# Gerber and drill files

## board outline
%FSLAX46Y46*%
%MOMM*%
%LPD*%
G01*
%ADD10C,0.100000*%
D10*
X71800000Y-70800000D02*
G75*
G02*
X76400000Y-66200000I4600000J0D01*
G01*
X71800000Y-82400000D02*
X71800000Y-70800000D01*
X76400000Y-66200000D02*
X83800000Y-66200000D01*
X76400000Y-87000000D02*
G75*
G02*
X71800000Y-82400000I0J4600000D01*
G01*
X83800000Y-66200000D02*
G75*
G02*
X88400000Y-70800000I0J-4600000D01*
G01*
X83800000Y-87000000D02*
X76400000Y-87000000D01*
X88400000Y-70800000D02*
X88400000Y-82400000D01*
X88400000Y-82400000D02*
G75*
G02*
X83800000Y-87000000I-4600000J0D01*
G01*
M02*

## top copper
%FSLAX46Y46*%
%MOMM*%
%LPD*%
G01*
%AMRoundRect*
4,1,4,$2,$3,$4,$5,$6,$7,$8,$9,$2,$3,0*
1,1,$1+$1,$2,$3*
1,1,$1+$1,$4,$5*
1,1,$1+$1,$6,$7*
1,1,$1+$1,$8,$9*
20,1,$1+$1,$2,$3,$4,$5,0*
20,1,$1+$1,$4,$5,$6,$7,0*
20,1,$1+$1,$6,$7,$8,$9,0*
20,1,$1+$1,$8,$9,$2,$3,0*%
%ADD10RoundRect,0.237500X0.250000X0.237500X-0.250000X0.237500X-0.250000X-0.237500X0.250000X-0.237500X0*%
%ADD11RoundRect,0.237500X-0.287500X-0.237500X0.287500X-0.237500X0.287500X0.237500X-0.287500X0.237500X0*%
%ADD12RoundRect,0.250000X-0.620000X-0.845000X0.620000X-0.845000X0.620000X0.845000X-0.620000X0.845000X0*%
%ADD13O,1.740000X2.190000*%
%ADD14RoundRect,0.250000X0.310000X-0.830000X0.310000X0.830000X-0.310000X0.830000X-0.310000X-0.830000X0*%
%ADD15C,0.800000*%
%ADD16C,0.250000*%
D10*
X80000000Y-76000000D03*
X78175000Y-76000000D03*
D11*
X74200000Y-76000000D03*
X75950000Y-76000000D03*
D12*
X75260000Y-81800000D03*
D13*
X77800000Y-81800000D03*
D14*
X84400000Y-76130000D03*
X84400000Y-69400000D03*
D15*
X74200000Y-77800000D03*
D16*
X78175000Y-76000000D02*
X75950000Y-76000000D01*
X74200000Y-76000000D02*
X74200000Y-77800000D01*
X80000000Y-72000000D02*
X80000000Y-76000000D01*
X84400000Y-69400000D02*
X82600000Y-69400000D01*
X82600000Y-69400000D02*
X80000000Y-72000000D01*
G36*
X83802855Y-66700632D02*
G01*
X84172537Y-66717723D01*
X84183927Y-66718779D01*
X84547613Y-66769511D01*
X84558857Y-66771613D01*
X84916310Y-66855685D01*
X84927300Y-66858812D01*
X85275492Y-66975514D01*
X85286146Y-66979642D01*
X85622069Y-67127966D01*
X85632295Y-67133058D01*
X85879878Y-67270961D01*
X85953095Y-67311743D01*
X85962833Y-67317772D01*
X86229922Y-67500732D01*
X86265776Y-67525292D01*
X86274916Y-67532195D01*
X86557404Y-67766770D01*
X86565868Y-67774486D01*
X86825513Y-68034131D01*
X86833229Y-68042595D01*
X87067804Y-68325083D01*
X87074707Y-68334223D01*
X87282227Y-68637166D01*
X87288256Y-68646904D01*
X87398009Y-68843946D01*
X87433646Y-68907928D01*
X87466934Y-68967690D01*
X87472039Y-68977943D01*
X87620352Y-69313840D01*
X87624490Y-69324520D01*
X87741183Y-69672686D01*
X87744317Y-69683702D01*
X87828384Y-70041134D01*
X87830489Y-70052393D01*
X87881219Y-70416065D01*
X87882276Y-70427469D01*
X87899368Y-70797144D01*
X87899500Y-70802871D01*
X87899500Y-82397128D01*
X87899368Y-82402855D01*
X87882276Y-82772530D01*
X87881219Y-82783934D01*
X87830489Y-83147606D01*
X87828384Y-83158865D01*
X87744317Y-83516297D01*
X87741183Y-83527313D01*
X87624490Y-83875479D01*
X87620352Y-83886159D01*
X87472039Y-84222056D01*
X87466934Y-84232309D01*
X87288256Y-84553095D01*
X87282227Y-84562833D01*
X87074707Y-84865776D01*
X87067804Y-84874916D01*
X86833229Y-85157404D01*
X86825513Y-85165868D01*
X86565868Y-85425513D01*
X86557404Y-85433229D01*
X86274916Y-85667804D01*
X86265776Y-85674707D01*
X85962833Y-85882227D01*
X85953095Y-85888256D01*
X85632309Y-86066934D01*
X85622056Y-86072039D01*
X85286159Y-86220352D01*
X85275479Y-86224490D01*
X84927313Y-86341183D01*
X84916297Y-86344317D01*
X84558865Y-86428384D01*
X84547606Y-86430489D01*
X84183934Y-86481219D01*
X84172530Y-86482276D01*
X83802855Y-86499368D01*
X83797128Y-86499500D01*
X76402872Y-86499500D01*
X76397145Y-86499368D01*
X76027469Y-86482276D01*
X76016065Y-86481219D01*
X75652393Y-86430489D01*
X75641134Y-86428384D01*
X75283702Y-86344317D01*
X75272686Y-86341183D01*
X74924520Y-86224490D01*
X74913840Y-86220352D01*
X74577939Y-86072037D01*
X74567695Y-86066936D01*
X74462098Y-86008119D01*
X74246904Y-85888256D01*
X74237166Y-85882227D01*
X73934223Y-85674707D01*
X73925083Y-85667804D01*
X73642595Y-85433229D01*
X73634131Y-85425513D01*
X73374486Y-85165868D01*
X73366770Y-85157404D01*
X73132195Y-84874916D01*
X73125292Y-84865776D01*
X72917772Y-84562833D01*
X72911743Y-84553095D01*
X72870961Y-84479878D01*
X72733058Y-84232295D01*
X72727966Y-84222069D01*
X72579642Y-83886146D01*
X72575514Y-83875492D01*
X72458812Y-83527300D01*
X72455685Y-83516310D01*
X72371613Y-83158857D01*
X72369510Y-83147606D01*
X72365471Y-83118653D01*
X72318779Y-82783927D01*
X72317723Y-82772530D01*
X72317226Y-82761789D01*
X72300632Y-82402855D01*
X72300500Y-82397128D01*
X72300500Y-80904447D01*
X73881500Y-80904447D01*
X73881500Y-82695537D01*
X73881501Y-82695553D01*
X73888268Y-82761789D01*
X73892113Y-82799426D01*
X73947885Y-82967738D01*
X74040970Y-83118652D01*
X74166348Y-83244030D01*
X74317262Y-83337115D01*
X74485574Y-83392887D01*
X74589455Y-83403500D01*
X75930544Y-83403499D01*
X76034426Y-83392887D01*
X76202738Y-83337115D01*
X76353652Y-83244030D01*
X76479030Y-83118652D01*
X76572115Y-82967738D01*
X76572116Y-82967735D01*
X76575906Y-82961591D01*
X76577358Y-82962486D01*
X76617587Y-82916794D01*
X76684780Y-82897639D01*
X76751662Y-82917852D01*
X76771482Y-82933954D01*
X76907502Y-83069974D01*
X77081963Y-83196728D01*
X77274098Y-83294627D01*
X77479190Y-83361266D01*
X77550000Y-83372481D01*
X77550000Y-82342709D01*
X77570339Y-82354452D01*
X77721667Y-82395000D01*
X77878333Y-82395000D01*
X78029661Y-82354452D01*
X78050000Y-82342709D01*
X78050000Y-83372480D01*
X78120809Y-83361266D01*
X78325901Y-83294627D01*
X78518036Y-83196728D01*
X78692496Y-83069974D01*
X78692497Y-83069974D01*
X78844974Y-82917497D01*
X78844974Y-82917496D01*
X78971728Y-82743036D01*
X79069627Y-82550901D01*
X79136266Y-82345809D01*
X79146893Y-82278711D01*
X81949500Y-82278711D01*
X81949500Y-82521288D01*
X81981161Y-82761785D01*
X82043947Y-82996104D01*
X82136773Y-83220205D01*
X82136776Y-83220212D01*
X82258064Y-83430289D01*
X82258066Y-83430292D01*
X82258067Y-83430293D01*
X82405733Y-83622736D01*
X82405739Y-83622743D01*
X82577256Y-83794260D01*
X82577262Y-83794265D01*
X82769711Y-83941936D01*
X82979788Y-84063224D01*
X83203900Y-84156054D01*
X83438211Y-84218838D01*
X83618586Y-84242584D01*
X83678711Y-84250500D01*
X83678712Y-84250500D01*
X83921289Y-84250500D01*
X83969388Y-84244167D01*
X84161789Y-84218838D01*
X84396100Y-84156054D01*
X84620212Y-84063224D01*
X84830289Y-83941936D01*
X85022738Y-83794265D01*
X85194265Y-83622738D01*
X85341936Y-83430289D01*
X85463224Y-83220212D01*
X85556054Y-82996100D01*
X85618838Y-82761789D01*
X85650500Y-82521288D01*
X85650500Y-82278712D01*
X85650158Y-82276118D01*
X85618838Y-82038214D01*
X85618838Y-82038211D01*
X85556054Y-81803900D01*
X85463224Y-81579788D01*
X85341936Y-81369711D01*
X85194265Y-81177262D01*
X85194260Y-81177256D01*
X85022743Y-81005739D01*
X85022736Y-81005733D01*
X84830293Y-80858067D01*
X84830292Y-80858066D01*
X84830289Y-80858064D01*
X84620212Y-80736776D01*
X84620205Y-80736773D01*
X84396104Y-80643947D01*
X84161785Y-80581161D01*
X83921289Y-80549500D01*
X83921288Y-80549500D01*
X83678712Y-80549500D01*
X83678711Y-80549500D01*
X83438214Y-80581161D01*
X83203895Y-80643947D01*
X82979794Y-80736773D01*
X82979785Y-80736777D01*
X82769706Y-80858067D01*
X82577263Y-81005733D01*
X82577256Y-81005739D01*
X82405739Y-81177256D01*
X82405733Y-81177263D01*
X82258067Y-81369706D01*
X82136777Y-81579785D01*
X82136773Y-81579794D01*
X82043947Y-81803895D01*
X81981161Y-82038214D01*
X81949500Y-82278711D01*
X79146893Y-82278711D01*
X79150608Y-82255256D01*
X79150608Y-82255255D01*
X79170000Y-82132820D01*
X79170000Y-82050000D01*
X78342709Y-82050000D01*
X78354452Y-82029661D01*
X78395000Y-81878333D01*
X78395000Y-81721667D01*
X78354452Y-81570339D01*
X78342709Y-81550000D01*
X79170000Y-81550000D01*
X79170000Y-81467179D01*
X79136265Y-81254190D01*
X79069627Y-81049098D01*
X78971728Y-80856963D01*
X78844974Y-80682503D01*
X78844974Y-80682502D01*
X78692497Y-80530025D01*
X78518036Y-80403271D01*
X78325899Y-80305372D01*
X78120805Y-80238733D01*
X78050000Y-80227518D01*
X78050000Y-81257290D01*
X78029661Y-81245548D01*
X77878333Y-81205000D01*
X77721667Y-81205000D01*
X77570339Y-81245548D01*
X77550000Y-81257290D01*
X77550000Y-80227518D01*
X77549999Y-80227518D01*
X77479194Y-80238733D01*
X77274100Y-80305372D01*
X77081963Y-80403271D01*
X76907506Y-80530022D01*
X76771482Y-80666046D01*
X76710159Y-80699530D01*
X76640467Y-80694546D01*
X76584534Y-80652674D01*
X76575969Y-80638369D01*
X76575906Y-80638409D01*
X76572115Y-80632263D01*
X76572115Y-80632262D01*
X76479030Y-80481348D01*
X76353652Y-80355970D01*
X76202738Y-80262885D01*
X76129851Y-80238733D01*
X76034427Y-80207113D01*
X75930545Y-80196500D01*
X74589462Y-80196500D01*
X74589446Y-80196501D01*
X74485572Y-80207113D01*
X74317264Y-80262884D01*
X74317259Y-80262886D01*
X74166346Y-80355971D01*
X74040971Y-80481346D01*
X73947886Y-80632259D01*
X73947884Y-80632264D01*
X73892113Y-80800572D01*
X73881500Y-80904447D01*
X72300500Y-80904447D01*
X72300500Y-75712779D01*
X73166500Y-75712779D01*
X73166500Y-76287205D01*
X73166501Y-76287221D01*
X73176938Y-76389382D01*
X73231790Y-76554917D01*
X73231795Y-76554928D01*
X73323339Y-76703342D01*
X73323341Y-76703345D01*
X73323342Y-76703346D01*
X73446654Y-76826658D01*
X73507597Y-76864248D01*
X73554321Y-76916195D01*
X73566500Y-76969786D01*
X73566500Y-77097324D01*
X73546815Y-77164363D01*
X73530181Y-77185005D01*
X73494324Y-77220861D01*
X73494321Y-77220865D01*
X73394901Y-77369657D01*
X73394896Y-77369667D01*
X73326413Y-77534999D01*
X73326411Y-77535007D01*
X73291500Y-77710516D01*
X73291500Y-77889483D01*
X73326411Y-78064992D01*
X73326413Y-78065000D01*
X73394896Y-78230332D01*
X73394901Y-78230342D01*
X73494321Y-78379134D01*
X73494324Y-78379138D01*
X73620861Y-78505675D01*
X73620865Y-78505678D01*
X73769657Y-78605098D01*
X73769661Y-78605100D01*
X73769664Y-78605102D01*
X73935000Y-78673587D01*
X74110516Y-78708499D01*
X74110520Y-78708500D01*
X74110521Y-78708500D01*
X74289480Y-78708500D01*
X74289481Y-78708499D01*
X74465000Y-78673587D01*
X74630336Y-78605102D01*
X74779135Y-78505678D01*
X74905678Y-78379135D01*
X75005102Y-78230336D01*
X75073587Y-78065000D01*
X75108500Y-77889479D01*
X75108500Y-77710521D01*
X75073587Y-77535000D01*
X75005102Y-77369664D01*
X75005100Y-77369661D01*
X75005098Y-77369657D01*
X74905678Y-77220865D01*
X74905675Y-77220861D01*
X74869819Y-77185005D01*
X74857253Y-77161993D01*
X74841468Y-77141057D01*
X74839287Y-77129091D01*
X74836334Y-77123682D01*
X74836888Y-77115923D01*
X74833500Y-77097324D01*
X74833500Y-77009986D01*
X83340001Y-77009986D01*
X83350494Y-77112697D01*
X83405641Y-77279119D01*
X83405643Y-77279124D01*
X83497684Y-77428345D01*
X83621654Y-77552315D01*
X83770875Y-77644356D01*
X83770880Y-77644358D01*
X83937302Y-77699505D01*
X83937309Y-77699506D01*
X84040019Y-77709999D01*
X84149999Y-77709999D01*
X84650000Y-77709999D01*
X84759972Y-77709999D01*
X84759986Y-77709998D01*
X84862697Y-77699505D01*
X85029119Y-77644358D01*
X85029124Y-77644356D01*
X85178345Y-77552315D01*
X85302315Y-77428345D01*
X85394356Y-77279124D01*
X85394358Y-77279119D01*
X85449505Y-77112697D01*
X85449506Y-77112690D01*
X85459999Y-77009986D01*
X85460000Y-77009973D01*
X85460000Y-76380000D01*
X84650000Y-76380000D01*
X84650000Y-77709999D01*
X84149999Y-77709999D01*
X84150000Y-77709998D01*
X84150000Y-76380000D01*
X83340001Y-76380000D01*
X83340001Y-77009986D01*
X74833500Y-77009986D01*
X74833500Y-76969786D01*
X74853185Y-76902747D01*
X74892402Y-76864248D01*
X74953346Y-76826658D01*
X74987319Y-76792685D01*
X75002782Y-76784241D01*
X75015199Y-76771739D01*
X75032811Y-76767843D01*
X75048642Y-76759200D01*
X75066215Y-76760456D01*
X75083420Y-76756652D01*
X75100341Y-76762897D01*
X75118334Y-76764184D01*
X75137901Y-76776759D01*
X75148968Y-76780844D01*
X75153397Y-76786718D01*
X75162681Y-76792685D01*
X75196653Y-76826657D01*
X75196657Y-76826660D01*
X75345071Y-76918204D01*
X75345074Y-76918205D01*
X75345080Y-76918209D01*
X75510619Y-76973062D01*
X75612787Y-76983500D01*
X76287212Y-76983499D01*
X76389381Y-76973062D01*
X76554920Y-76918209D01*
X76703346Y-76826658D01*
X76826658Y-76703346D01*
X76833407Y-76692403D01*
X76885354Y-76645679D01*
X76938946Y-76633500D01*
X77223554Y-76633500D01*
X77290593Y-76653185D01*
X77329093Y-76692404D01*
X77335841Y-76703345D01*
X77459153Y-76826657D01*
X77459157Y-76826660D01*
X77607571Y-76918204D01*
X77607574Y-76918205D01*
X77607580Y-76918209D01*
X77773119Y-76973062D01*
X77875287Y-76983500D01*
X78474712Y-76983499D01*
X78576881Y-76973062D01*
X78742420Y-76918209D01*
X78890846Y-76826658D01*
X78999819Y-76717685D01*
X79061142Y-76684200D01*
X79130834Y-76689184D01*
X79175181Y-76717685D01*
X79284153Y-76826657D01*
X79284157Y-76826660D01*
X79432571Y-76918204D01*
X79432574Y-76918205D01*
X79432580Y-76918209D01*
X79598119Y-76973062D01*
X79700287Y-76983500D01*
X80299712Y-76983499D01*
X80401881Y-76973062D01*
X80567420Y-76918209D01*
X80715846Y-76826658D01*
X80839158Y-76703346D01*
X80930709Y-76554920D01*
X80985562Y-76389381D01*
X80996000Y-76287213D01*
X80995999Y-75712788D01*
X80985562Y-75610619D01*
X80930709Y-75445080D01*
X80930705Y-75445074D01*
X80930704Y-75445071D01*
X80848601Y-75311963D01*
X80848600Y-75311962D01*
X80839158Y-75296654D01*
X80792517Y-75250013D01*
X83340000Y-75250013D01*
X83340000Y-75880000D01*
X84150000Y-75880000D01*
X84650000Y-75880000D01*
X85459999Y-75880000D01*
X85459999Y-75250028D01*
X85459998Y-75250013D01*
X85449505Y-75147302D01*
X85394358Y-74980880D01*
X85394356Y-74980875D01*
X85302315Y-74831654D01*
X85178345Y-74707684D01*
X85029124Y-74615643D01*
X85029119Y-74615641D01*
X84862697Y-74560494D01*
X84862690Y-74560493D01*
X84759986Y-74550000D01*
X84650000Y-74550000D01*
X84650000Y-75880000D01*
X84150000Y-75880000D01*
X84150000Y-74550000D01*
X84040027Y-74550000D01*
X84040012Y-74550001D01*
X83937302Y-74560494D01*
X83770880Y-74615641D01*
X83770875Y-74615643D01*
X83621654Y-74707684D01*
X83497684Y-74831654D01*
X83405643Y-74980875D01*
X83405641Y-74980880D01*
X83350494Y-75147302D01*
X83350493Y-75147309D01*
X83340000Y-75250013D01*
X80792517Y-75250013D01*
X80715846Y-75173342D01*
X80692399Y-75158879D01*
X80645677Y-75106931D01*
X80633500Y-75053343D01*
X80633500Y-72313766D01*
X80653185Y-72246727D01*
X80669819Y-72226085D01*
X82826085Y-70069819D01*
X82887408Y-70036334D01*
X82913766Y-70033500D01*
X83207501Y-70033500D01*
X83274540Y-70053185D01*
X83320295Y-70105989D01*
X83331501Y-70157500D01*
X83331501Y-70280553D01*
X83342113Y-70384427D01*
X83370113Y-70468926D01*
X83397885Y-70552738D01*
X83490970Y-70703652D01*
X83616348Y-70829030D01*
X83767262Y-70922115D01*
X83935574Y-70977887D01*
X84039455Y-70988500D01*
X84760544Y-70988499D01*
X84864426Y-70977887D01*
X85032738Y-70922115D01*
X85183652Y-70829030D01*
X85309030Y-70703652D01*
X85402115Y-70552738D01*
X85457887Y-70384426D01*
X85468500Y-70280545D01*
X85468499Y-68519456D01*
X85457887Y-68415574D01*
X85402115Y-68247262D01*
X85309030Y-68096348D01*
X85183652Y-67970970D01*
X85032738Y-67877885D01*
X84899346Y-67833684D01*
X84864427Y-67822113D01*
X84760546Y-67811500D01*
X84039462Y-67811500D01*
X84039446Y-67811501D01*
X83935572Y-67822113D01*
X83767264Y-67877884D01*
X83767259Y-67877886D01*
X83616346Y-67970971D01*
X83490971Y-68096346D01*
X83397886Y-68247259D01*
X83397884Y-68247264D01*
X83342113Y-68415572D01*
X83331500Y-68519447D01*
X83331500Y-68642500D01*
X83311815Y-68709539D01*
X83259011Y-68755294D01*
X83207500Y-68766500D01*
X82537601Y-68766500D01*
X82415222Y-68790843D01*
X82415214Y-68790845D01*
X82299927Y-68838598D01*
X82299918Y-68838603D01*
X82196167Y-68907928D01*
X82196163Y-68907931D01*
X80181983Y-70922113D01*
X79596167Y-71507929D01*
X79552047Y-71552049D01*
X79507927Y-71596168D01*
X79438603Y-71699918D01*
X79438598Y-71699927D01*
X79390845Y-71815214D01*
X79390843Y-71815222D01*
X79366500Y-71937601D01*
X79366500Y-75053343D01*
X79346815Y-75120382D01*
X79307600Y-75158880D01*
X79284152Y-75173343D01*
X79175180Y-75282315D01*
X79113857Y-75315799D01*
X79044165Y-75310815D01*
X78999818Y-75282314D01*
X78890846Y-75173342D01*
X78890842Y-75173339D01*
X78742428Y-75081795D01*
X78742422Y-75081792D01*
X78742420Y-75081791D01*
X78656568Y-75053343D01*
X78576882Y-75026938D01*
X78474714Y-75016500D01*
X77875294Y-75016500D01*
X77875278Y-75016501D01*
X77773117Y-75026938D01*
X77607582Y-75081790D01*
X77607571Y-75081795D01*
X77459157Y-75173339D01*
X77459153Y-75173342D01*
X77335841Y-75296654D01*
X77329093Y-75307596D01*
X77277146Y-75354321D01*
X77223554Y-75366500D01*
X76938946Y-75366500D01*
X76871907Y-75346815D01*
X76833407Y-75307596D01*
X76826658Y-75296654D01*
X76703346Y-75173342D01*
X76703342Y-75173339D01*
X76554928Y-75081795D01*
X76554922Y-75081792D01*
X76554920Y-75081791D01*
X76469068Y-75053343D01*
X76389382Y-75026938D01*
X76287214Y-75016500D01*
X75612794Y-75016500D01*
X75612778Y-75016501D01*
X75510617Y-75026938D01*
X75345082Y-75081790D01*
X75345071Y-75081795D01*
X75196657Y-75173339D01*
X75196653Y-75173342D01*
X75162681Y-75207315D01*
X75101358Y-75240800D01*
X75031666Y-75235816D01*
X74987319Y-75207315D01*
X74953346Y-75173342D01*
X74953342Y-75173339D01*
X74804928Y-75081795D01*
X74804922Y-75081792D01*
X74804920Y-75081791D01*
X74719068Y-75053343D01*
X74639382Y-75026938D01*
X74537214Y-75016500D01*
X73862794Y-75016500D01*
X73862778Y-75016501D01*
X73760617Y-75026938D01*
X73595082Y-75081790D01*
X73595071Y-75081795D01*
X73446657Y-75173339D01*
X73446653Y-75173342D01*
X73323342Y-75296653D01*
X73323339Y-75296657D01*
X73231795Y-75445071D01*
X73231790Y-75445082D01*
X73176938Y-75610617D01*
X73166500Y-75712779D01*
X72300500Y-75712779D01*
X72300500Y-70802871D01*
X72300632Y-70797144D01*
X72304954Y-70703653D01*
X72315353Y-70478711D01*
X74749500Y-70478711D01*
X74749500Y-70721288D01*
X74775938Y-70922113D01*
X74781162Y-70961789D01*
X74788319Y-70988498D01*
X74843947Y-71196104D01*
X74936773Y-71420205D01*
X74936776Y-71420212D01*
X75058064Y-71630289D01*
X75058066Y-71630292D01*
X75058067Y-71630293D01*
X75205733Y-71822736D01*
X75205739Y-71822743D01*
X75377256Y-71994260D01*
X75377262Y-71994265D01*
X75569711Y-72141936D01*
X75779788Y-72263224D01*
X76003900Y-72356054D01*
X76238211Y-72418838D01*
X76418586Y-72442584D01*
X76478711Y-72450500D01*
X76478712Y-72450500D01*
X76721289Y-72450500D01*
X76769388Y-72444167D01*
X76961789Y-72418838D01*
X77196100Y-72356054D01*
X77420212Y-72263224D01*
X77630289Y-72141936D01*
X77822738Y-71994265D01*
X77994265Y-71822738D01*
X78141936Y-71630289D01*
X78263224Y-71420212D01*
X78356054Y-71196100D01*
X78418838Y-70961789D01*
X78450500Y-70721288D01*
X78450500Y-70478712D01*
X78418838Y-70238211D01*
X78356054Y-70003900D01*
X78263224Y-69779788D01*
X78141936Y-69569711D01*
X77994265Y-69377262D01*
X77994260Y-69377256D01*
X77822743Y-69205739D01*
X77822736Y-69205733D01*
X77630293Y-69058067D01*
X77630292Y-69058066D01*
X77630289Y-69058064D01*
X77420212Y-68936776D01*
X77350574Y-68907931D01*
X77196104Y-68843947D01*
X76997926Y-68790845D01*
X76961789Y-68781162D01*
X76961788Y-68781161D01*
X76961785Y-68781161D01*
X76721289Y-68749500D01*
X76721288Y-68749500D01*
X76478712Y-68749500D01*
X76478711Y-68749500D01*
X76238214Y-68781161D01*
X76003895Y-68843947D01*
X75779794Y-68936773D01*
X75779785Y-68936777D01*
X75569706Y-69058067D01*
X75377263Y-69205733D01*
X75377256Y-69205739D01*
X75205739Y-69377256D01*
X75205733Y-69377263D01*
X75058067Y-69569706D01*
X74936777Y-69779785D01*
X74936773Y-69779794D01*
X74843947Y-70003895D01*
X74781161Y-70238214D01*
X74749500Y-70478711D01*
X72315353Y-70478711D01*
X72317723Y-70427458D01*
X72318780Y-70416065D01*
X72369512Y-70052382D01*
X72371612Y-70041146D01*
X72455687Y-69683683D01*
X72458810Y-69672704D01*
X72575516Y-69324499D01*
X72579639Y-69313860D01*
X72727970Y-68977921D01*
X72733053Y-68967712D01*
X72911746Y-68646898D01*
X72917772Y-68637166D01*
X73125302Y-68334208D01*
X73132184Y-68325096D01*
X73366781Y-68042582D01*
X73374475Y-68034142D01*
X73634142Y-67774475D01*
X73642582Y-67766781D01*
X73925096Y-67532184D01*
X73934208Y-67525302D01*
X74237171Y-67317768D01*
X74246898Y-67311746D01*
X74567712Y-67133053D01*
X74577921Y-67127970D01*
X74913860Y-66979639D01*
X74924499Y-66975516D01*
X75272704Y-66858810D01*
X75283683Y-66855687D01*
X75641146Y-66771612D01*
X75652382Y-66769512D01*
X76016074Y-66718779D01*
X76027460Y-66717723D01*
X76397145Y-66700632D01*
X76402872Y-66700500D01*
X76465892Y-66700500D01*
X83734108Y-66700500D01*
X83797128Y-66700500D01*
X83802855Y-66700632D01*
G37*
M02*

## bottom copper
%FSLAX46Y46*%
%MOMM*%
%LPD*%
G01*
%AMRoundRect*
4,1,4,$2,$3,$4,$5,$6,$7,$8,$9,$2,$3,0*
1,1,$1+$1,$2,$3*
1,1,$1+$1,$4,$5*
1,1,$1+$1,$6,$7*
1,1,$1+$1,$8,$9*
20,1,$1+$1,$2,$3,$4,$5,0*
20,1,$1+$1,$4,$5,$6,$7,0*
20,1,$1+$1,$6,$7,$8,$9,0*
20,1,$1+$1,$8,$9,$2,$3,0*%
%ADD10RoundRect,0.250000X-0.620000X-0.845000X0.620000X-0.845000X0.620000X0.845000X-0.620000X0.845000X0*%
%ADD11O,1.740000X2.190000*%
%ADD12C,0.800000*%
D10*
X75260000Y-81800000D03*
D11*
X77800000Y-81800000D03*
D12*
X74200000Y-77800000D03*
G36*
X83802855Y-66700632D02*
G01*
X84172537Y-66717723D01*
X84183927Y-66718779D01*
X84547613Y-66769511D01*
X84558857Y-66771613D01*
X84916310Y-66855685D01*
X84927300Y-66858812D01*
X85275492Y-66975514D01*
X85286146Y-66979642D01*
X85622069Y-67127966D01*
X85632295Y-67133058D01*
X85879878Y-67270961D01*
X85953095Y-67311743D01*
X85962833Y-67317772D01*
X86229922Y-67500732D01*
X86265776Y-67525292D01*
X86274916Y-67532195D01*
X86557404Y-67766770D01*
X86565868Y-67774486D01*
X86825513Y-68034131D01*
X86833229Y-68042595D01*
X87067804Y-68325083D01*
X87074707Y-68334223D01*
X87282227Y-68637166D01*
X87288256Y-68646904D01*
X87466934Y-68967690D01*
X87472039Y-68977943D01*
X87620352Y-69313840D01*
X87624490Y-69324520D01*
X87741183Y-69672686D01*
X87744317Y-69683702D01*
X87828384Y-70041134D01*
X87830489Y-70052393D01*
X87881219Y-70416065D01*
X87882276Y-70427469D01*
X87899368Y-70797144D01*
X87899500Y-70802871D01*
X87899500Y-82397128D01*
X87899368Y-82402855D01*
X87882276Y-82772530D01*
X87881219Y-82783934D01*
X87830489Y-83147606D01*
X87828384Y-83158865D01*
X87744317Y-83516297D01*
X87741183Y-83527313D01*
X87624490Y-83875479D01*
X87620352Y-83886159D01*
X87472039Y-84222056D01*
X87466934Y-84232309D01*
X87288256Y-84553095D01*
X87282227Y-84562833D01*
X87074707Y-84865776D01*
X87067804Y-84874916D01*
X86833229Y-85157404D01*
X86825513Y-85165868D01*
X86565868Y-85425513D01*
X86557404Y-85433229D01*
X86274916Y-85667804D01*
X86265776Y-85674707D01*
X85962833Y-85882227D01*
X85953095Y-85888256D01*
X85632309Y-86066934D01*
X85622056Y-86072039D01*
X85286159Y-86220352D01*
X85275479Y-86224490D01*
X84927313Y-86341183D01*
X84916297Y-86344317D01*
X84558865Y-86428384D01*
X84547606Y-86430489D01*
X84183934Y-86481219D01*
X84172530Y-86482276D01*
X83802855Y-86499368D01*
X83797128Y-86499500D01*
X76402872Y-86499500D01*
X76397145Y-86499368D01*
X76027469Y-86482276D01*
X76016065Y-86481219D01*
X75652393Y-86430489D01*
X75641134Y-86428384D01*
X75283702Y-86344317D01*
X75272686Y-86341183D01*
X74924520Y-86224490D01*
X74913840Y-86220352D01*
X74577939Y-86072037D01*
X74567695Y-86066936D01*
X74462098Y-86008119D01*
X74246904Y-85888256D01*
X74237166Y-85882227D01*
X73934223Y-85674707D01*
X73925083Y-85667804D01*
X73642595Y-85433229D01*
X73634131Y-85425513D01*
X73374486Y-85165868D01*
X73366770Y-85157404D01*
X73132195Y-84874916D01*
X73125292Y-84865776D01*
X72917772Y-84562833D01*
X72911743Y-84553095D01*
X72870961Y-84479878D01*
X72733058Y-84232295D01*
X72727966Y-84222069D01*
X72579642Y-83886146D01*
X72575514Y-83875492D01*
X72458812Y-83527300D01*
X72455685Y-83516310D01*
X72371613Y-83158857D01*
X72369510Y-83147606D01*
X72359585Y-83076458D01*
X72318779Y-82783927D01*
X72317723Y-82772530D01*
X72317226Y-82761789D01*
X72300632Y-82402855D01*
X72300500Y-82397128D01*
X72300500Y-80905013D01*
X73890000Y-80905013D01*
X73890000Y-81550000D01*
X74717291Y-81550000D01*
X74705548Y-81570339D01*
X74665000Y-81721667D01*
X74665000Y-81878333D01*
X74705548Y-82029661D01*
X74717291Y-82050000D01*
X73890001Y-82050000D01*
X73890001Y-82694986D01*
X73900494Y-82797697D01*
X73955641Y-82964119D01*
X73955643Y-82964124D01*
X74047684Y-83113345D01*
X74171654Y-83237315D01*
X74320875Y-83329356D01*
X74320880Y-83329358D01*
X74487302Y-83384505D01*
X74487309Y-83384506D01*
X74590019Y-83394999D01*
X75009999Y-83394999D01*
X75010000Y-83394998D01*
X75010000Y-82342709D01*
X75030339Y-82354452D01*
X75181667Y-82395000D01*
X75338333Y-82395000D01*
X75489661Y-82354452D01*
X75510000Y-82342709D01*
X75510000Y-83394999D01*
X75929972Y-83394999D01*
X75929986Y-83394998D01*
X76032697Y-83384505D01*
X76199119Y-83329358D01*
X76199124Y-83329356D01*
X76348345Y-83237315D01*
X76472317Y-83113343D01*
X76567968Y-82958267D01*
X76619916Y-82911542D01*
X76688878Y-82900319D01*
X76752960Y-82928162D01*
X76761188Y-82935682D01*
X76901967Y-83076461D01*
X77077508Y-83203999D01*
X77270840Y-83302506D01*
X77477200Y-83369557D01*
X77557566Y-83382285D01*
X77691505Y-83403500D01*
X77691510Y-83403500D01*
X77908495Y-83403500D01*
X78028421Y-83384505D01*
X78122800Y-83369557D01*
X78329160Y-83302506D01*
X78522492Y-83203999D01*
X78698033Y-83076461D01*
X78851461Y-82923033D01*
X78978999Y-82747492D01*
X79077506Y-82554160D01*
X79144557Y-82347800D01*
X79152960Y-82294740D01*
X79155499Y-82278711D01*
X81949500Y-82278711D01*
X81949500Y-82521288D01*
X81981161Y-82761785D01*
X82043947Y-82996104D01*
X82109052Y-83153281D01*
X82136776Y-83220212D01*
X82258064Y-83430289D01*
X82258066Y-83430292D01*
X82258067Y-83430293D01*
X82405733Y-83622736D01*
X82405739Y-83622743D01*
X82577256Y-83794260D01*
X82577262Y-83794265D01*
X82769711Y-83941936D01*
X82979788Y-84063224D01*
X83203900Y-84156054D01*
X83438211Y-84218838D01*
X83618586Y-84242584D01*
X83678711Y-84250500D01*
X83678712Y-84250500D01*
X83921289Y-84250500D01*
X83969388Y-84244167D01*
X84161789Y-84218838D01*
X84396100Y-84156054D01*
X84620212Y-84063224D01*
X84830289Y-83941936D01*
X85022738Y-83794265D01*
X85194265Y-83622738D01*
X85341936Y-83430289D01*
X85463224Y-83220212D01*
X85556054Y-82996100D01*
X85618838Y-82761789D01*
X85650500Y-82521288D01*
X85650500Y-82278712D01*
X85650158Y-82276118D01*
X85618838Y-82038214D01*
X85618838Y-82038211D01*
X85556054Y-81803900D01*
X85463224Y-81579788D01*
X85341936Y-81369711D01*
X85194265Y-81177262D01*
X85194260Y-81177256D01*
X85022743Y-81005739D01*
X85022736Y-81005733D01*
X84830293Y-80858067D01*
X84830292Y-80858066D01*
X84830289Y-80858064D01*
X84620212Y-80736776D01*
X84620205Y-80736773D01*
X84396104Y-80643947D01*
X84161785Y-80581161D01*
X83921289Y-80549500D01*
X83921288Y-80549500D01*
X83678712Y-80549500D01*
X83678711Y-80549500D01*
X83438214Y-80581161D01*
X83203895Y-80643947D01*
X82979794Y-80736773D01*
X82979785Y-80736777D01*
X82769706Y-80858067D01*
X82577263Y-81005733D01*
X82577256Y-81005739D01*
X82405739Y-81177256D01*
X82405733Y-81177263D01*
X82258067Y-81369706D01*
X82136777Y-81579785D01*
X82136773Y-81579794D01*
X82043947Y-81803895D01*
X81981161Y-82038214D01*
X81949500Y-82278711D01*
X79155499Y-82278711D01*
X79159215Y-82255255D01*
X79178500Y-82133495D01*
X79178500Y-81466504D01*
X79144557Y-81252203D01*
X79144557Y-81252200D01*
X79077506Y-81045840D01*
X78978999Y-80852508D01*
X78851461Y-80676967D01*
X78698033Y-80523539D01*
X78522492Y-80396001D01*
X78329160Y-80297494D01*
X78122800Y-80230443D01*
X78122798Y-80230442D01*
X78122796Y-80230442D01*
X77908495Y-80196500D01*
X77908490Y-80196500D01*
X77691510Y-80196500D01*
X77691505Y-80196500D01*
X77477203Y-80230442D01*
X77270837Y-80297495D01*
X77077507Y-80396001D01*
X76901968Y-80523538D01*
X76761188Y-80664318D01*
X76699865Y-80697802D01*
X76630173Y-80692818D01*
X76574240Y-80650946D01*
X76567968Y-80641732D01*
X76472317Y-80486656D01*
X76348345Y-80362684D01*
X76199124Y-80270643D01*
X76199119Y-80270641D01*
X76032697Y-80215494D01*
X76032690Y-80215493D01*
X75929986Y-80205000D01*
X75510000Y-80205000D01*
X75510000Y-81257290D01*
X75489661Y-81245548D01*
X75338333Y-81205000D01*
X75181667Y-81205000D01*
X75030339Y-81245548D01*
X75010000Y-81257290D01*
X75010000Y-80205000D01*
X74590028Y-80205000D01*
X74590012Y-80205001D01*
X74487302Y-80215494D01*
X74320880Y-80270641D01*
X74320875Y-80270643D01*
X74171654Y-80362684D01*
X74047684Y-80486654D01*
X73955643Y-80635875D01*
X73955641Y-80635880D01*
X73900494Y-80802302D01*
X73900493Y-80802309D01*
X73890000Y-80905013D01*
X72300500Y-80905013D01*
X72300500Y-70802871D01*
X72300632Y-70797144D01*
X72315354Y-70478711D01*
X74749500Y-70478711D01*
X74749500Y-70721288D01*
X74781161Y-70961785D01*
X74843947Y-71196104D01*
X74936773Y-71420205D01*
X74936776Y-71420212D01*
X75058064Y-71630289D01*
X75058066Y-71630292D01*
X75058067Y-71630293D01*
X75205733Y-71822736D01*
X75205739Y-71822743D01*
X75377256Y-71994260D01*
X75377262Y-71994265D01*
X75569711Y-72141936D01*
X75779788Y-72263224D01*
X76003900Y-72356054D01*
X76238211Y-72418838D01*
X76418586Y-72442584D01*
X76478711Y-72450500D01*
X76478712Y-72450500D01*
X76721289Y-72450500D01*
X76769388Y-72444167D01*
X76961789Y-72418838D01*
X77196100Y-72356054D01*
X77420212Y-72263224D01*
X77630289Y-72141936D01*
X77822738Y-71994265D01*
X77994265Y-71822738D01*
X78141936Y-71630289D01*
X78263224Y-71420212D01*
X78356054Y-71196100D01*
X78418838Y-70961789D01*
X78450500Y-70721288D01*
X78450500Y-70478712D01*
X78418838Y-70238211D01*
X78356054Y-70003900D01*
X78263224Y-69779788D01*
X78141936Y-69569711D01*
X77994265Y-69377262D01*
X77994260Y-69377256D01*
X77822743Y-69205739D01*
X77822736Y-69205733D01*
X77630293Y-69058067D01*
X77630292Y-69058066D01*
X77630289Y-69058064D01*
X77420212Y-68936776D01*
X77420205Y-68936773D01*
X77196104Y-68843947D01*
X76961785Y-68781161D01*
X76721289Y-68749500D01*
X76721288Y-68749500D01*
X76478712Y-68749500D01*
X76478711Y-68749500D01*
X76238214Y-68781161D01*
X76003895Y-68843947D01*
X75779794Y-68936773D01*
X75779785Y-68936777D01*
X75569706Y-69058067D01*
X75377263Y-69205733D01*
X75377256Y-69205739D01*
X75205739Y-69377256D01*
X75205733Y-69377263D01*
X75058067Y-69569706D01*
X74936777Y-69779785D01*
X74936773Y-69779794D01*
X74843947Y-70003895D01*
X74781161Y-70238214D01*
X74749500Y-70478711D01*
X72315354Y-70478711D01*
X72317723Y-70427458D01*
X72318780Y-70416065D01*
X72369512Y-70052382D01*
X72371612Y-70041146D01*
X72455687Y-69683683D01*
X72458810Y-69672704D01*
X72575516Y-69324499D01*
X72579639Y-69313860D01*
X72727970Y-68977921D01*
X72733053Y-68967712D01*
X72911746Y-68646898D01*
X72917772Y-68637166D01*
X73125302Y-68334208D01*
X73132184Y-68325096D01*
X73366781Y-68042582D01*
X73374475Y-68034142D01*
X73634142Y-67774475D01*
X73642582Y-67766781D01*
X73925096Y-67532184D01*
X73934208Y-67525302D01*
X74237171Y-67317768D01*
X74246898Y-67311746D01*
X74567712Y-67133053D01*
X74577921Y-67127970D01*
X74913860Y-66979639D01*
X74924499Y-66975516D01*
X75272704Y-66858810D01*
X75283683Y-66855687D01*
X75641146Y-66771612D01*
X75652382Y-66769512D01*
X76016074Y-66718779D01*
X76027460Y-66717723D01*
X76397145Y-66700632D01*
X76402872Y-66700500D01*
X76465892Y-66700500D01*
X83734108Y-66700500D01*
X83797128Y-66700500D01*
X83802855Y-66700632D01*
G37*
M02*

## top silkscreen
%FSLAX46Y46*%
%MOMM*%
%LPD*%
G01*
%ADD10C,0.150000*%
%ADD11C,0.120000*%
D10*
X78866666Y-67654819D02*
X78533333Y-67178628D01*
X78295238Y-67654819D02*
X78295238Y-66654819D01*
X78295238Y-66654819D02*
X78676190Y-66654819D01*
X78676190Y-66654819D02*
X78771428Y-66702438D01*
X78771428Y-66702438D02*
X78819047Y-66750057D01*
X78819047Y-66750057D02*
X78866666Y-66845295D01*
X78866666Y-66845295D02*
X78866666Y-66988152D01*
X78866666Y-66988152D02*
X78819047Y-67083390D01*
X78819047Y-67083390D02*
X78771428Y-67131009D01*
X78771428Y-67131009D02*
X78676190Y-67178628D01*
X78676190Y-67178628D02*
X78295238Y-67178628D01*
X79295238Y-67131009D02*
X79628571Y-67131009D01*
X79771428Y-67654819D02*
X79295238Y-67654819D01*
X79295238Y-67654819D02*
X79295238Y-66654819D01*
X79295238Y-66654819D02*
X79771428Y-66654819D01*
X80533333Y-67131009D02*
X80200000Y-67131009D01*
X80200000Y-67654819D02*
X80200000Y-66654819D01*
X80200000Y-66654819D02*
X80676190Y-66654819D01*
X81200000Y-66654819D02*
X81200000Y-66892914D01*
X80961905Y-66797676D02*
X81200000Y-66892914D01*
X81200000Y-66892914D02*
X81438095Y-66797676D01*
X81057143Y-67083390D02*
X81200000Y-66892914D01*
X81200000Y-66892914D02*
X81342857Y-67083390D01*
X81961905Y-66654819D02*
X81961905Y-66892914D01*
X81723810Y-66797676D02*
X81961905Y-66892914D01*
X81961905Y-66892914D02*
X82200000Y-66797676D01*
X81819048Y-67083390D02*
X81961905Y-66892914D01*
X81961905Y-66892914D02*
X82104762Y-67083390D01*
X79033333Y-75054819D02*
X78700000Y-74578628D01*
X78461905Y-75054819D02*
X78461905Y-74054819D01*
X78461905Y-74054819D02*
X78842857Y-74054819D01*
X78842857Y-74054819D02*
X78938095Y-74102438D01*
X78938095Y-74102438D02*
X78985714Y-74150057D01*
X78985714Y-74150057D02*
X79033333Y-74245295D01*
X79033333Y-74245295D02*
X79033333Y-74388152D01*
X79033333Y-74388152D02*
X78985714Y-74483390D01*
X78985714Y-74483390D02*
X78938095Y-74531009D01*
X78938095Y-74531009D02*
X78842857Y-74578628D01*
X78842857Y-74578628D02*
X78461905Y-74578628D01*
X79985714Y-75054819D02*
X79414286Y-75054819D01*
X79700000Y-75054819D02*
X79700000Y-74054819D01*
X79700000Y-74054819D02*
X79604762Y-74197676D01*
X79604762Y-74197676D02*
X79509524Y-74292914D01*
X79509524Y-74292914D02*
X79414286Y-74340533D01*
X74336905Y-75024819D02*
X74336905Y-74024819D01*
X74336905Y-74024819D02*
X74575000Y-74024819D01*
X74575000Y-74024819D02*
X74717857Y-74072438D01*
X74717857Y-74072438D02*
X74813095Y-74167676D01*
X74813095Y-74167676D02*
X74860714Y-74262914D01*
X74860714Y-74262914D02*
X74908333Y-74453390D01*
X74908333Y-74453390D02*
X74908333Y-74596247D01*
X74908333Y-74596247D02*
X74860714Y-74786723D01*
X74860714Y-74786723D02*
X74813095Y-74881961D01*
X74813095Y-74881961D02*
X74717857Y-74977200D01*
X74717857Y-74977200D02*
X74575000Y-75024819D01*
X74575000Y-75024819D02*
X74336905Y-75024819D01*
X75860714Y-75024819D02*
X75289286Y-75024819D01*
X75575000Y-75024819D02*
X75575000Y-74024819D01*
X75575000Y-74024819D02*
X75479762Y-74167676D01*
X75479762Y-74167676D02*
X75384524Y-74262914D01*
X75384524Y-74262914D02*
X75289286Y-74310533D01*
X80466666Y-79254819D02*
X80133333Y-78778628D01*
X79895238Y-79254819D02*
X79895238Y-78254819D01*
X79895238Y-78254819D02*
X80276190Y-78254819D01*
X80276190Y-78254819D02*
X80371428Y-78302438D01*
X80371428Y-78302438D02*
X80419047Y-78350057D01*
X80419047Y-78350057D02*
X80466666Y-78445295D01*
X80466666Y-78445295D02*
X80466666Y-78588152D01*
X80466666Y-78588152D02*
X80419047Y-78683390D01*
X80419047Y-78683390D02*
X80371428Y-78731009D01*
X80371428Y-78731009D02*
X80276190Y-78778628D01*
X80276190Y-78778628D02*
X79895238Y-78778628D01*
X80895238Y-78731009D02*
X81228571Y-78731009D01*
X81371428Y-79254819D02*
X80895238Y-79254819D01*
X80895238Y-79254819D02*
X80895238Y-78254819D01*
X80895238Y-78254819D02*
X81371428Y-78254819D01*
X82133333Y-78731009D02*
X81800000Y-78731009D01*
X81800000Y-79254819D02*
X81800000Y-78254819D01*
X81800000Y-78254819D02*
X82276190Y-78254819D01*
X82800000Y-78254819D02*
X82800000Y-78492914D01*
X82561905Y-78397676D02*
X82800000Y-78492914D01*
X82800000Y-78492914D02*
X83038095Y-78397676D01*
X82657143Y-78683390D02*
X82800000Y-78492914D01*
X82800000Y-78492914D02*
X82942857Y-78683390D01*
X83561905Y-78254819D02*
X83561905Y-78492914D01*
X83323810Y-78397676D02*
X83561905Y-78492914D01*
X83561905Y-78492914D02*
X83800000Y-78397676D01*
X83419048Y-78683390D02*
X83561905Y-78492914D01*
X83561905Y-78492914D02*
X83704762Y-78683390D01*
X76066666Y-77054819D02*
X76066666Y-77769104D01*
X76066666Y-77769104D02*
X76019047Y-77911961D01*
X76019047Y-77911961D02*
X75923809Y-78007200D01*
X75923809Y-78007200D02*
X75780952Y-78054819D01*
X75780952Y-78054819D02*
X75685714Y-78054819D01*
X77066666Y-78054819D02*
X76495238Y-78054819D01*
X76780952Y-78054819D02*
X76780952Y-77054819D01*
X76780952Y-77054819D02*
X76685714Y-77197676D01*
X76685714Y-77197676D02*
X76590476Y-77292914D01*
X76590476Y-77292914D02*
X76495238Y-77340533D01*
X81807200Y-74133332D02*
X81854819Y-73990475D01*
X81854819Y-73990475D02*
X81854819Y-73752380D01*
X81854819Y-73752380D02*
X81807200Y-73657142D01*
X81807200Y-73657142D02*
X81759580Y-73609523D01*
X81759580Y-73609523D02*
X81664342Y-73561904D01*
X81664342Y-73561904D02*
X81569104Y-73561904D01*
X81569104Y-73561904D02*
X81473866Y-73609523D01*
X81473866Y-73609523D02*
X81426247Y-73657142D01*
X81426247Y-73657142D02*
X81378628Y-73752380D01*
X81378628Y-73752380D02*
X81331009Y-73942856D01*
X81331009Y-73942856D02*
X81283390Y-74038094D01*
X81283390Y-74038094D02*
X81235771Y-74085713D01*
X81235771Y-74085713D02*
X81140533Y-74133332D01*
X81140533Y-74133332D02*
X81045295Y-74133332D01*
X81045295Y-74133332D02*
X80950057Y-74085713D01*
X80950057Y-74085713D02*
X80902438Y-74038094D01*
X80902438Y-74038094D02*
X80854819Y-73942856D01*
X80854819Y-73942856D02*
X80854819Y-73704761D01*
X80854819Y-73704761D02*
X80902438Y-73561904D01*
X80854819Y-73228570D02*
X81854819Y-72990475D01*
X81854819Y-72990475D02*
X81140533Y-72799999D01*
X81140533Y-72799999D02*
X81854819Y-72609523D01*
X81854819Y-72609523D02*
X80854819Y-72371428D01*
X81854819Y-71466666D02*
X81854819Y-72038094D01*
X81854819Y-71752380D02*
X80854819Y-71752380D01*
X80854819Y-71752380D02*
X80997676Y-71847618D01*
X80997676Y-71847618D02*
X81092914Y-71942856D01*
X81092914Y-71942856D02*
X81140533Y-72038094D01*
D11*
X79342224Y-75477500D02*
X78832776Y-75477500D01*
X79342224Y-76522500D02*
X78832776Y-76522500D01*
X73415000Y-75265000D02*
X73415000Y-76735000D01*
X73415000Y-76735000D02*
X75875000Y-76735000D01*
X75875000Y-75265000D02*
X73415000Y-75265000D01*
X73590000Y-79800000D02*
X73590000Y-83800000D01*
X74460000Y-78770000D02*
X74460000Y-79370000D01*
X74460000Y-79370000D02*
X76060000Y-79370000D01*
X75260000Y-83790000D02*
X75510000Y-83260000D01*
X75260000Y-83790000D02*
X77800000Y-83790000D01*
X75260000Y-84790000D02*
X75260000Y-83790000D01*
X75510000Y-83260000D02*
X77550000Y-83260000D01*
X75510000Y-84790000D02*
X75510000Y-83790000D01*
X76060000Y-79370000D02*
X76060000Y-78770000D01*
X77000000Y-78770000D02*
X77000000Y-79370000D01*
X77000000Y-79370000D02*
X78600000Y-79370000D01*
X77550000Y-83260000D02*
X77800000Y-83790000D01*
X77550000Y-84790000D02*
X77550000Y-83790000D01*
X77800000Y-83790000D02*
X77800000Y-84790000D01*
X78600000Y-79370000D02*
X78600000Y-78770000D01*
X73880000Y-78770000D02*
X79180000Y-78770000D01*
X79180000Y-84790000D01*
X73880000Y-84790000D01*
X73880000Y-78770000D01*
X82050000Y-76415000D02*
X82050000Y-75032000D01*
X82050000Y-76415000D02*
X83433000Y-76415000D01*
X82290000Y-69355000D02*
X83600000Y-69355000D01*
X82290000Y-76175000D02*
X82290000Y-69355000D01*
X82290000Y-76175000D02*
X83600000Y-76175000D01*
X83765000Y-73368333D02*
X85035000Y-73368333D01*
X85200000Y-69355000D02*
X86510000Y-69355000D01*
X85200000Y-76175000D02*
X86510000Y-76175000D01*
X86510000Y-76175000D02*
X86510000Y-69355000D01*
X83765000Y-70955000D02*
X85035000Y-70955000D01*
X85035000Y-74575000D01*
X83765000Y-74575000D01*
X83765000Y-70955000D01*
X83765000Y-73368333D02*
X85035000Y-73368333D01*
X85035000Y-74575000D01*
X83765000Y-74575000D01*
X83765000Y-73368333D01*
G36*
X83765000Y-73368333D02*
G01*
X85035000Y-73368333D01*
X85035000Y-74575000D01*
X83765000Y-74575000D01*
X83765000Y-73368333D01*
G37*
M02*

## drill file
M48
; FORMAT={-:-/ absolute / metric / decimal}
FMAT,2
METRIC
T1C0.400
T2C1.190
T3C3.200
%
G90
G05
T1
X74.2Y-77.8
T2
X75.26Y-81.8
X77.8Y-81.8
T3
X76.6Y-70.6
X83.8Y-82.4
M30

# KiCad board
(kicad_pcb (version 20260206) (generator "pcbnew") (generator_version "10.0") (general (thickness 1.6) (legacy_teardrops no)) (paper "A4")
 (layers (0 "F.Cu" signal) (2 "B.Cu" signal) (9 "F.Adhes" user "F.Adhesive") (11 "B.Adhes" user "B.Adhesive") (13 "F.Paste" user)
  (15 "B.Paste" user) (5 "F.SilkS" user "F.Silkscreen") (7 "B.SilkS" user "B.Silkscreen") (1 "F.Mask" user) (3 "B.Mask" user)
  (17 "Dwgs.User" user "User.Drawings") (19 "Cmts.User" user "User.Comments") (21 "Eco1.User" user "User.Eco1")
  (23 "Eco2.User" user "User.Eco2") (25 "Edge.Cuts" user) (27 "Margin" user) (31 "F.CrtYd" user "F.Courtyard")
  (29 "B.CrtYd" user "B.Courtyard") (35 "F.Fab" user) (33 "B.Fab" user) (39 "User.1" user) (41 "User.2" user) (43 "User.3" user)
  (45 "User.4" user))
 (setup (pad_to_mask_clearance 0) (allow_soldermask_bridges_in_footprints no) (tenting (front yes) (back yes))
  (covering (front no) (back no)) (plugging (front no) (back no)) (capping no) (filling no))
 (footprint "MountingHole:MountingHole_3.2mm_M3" (layer "F.Cu") (at 76.6 70.6)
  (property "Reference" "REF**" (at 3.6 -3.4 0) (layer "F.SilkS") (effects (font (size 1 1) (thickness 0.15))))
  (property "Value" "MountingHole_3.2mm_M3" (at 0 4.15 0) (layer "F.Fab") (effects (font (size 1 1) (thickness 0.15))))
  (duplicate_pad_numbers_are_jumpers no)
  (pad "" np_thru_hole circle (at 0 0) (size 3.2 3.2) (drill 3.2) (layers "*.Cu" "*.Mask")))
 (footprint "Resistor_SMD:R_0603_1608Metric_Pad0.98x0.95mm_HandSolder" (layer "F.Cu") (at 79.0875 76 180)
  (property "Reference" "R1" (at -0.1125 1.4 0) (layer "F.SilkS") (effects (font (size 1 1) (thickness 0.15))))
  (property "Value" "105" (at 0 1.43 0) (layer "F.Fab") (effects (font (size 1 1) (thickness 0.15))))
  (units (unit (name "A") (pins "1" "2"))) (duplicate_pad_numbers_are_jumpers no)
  (fp_line (start -0.254724 0.5225) (end 0.254724 0.5225) (stroke (width 0.12) (type solid)) (layer "F.SilkS"))
  (fp_line (start -0.254724 -0.5225) (end 0.254724 -0.5225) (stroke (width 0.12) (type solid)) (layer "F.SilkS"))
  (pad "1" smd roundrect (at -0.9125 0 180) (size 0.975 0.95) (layers "F.Cu" "F.Mask" "F.Paste") (roundrect_rratio 0.25)
   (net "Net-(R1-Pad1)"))
  (pad "2" smd roundrect (at 0.9125 0 180) (size 0.975 0.95) (layers "F.Cu" "F.Mask" "F.Paste") (roundrect_rratio 0.25) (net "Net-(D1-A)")))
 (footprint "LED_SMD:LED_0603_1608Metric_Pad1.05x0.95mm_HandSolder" (layer "F.Cu") (at 75.075 76)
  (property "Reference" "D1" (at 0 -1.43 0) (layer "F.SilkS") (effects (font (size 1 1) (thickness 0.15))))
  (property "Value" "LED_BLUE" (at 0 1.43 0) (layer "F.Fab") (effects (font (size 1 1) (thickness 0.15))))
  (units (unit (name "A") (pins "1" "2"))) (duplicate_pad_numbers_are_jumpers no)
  (fp_line (start -1.66 -0.735) (end -1.66 0.735) (stroke (width 0.12) (type solid)) (layer "F.SilkS"))
  (fp_line (start -1.66 0.735) (end 0.8 0.735) (stroke (width 0.12) (type solid)) (layer "F.SilkS"))
  (fp_line (start 0.8 -0.735) (end -1.66 -0.735) (stroke (width 0.12) (type solid)) (layer "F.SilkS"))
  (pad "1" smd roundrect (at -0.875 0) (size 1.05 0.95) (layers "F.Cu" "F.Mask" "F.Paste") (roundrect_rratio 0.25) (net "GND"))
  (pad "2" smd roundrect (at 0.875 0) (size 1.05 0.95) (layers "F.Cu" "F.Mask" "F.Paste") (roundrect_rratio 0.25) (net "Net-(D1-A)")))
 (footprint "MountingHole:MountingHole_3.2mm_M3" (layer "F.Cu") (at 83.8 82.4)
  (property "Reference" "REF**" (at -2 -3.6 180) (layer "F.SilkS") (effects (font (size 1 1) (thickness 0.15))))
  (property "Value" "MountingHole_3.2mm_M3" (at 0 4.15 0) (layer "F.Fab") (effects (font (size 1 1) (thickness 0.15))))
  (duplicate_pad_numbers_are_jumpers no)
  (pad "" np_thru_hole circle (at 0 0) (size 3.2 3.2) (drill 3.2) (layers "*.Cu" "*.Mask")))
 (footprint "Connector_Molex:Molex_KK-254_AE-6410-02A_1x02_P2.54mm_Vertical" (layer "F.Cu") (at 75.26 81.8)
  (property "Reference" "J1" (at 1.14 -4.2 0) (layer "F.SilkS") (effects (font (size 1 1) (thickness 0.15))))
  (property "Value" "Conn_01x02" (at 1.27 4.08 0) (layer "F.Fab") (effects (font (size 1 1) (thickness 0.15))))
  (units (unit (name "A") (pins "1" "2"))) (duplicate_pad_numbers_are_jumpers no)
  (fp_line (start -1.67 -2) (end -1.67 2) (stroke (width 0.12) (type solid)) (layer "F.SilkS"))
  (fp_line (start -0.8 -3.03) (end -0.8 -2.43) (stroke (width 0.12) (type solid)) (layer "F.SilkS"))
  (fp_line (start -0.8 -2.43) (end 0.8 -2.43) (stroke (width 0.12) (type solid)) (layer "F.SilkS"))
  (fp_line (start 0 1.99) (end 0.25 1.46) (stroke (width 0.12) (type solid)) (layer "F.SilkS"))
  (fp_line (start 0 1.99) (end 2.54 1.99) (stroke (width 0.12) (type solid)) (layer "F.SilkS"))
  (fp_line (start 0 2.99) (end 0 1.99) (stroke (width 0.12) (type solid)) (layer "F.SilkS"))
  (fp_line (start 0.25 1.46) (end 2.29 1.46) (stroke (width 0.12) (type solid)) (layer "F.SilkS"))
  (fp_line (start 0.25 2.99) (end 0.25 1.99) (stroke (width 0.12) (type solid)) (layer "F.SilkS"))
  (fp_line (start 0.8 -2.43) (end 0.8 -3.03) (stroke (width 0.12) (type solid)) (layer "F.SilkS"))
  (fp_line (start 1.74 -3.03) (end 1.74 -2.43) (stroke (width 0.12) (type solid)) (layer "F.SilkS"))
  (fp_line (start 1.74 -2.43) (end 3.34 -2.43) (stroke (width 0.12) (type solid)) (layer "F.SilkS"))
  (fp_line (start 2.29 1.46) (end 2.54 1.99) (stroke (width 0.12) (type solid)) (layer "F.SilkS"))
  (fp_line (start 2.29 2.99) (end 2.29 1.99) (stroke (width 0.12) (type solid)) (layer "F.SilkS"))
  (fp_line (start 2.54 1.99) (end 2.54 2.99) (stroke (width 0.12) (type solid)) (layer "F.SilkS"))
  (fp_line (start 3.34 -2.43) (end 3.34 -3.03) (stroke (width 0.12) (type solid)) (layer "F.SilkS"))
  (fp_rect (start -1.38 -3.03) (end 3.92 2.99) (stroke (width 0.12) (type solid)) (fill no) (layer "F.SilkS"))
  (pad "1" thru_hole roundrect (at 0 0) (size 1.74 2.19) (drill 1.19) (layers "*.Cu" "*.Mask") (remove_unused_layers no)
   (roundrect_rratio 0.143678) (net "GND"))
  (pad "2" thru_hole oval (at 2.54 0) (size 1.74 2.19) (drill 1.19) (layers "*.Cu" "*.Mask") (remove_unused_layers no) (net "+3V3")))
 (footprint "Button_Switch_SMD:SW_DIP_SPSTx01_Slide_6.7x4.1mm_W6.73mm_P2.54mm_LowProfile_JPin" (layer "F.Cu") (at 84.4 72.765 90)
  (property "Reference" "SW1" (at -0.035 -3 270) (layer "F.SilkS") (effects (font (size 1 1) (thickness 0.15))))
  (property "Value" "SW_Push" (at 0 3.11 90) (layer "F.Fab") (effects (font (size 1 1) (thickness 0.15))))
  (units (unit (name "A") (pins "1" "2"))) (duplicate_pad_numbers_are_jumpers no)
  (fp_line (start -3.65 -2.35) (end -2.267 -2.35) (stroke (width 0.12) (type solid)) (layer "F.SilkS"))
  (fp_line (start -3.65 -2.35) (end -3.65 -0.967) (stroke (width 0.12) (type solid)) (layer "F.SilkS"))
  (fp_line (start 3.41 -2.11) (end 3.41 -0.8) (stroke (width 0.12) (type solid)) (layer "F.SilkS"))
  (fp_line (start -3.41 -2.11) (end 3.41 -2.11) (stroke (width 0.12) (type solid)) (layer "F.SilkS"))
  (fp_line (start -3.41 -2.11) (end -3.41 -0.8) (stroke (width 0.12) (type solid)) (layer "F.SilkS"))
  (fp_line (start -0.603333 -0.635) (end -0.603333 0.635) (stroke (width 0.12) (type solid)) (layer "F.SilkS"))
  (fp_line (start 3.41 0.8) (end 3.41 2.11) (stroke (width 0.12) (type solid)) (layer "F.SilkS"))
  (fp_line (start -3.41 0.8) (end -3.41 2.11) (stroke (width 0.12) (type solid)) (layer "F.SilkS"))
  (fp_line (start -3.41 2.11) (end 3.41 2.11) (stroke (width 0.12) (type solid)) (layer "F.SilkS"))
  (fp_rect (start -1.81 -0.635) (end 1.81 0.635) (stroke (width 0.12) (type solid)) (fill no) (layer "F.SilkS"))
  (fp_rect (start -1.81 -0.635) (end -0.603333 0.635) (stroke (width 0.12) (type solid)) (fill yes) (layer "F.SilkS"))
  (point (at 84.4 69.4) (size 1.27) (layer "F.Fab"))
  (pad "1" smd roundrect (at -3.365 0 90) (size 2.16 1.12) (layers "F.Cu" "F.Mask" "F.Paste") (roundrect_rratio 0.223214) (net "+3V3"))
  (pad "2" smd roundrect (at 3.365 0 90) (size 2.16 1.12) (layers "F.Cu" "F.Mask" "F.Paste") (roundrect_rratio 0.223214)
   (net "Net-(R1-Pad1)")))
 (gr_arc (start 71.8 70.8) (mid 73.147309 67.547309) (end 76.4 66.2) (stroke (width 0.1) (type default)) (layer "Edge.Cuts"))
 (gr_line (start 71.8 82.4) (end 71.8 70.8) (stroke (width 0.1) (type default)) (layer "Edge.Cuts"))
 (gr_line (start 76.4 66.2) (end 83.8 66.2) (stroke (width 0.1) (type default)) (layer "Edge.Cuts"))
 (gr_arc (start 76.4 87) (mid 73.147309 85.652691) (end 71.8 82.4) (stroke (width 0.1) (type default)) (layer "Edge.Cuts"))
 (gr_arc (start 83.8 66.2) (mid 87.052691 67.547309) (end 88.4 70.8) (stroke (width 0.1) (type default)) (layer "Edge.Cuts"))
 (gr_line (start 83.8 87) (end 76.4 87) (stroke (width 0.1) (type default)) (layer "Edge.Cuts"))
 (gr_line (start 88.4 70.8) (end 88.4 82.4) (stroke (width 0.1) (type default)) (layer "Edge.Cuts"))
 (gr_arc (start 88.4 82.4) (mid 87.052691 85.652691) (end 83.8 87) (stroke (width 0.1) (type default)) (layer "Edge.Cuts"))
 (segment (start 78.175 76) (end 75.95 76) (width 0.25) (layer "F.Cu") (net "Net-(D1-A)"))
 (segment (start 74.2 76) (end 74.2 77.8) (width 0.25) (layer "F.Cu") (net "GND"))
 (via (at 74.2 77.8) (size 0.8) (drill 0.4) (layers "F.Cu" "B.Cu") (free yes) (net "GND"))
 (segment (start 80 72) (end 80 76) (width 0.25) (layer "F.Cu") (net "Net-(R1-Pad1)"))
 (segment (start 84.4 69.4) (end 82.6 69.4) (width 0.25) (layer "F.Cu") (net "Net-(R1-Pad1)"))
 (segment (start 82.6 69.4) (end 80 72) (width 0.25) (layer "F.Cu") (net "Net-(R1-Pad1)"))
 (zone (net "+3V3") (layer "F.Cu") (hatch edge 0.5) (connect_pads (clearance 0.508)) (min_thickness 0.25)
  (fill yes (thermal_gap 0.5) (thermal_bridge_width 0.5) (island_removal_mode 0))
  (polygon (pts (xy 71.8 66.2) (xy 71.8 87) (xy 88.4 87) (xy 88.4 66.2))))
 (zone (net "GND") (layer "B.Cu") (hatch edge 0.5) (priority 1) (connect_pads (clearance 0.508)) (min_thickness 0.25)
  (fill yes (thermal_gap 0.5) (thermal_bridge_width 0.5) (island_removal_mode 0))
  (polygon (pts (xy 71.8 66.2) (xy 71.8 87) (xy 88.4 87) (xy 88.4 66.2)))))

